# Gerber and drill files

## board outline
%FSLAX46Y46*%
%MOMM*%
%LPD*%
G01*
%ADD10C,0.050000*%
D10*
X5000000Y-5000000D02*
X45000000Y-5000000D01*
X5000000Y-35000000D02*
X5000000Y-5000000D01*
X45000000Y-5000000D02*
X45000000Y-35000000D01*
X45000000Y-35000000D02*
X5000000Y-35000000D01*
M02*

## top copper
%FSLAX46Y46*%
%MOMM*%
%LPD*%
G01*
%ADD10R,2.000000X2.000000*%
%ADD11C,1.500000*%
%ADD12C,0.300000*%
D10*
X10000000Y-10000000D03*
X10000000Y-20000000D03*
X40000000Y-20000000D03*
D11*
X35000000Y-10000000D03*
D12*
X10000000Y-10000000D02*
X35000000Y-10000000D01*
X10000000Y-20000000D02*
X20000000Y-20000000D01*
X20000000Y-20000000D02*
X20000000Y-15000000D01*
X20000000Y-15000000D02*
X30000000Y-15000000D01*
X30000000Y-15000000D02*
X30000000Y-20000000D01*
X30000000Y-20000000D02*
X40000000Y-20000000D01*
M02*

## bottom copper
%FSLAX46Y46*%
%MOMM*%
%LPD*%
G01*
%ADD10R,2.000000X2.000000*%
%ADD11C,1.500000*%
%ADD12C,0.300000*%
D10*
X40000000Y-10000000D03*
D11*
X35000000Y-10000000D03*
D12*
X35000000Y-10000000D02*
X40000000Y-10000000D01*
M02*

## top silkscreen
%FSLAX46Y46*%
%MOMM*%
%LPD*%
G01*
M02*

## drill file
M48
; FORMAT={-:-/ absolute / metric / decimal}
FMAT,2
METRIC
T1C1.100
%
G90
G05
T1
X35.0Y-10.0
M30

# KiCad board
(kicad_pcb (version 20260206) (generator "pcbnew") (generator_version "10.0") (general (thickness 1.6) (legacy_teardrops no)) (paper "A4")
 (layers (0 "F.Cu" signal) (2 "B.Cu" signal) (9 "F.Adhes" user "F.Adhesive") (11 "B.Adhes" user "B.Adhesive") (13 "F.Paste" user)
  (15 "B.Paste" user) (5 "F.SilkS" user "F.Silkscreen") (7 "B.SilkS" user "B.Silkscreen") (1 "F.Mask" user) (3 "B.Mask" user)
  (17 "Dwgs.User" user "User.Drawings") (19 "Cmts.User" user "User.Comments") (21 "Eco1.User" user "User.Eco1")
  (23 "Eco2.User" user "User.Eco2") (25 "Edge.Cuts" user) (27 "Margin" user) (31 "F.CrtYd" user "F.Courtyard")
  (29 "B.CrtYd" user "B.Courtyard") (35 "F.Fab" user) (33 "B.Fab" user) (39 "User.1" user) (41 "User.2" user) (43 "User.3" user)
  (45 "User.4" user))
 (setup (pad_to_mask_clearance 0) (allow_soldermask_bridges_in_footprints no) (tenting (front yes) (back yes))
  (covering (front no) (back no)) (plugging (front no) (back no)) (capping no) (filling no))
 (gr_line (start 5 5) (end 45 5) (stroke (width 0.05) (type default)) (layer "Edge.Cuts"))
 (gr_line (start 5 35) (end 5 5) (stroke (width 0.05) (type default)) (layer "Edge.Cuts"))
 (gr_line (start 45 5) (end 45 35) (stroke (width 0.05) (type default)) (layer "Edge.Cuts"))
 (gr_line (start 45 35) (end 5 35) (stroke (width 0.05) (type default)) (layer "Edge.Cuts"))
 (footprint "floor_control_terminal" (layer "F.Cu") (at 10 10)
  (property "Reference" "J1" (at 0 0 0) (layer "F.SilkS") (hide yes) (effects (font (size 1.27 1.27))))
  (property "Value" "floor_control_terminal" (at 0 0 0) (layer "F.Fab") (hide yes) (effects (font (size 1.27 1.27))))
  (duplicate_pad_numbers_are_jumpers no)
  (pad "1" smd rect (at 0 0) (size 2 2) (layers "F.Cu" "F.Paste" "F.Mask") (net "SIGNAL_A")))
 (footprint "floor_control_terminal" (layer "B.Cu") (at 40 10)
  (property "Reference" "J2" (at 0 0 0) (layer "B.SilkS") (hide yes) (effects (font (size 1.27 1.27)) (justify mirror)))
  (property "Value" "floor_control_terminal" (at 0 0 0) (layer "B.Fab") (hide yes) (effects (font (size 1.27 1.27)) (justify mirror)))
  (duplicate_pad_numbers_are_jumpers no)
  (pad "1" smd rect (at 0 0) (size 2 2) (layers "B.Cu" "B.Paste" "B.Mask") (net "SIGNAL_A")))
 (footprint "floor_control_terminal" (layer "F.Cu") (at 10 20)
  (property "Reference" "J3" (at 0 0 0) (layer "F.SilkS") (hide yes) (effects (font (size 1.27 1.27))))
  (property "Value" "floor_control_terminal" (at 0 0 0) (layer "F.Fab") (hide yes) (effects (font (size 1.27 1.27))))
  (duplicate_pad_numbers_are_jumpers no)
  (pad "1" smd rect (at 0 0) (size 2 2) (layers "F.Cu" "F.Paste" "F.Mask") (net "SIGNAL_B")))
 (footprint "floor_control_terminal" (layer "F.Cu") (at 40 20)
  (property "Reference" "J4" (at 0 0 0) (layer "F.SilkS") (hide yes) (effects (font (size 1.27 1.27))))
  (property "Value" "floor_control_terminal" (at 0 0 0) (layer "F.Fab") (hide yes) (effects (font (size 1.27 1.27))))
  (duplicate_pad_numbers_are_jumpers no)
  (pad "1" smd rect (at 0 0) (size 2 2) (layers "F.Cu" "F.Paste" "F.Mask") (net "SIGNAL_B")))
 (segment (start 10 10) (end 35 10) (width 0.3) (layer "F.Cu") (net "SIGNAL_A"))
 (segment (start 35 10) (end 40 10) (width 0.3) (layer "B.Cu") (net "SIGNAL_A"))
 (via (at 35 10) (size 1.5) (drill 1.1) (layers "F.Cu" "B.Cu") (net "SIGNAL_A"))
 (segment (start 10 20) (end 20 20) (width 0.3) (layer "F.Cu") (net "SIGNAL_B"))
 (segment (start 20 20) (end 20 15) (width 0.3) (layer "F.Cu") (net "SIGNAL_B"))
 (segment (start 20 15) (end 30 15) (width 0.3) (layer "F.Cu") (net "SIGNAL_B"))
 (segment (start 30 15) (end 30 20) (width 0.3) (layer "F.Cu") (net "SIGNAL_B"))
 (segment (start 30 20) (end 40 20) (width 0.3) (layer "F.Cu") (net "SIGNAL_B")))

